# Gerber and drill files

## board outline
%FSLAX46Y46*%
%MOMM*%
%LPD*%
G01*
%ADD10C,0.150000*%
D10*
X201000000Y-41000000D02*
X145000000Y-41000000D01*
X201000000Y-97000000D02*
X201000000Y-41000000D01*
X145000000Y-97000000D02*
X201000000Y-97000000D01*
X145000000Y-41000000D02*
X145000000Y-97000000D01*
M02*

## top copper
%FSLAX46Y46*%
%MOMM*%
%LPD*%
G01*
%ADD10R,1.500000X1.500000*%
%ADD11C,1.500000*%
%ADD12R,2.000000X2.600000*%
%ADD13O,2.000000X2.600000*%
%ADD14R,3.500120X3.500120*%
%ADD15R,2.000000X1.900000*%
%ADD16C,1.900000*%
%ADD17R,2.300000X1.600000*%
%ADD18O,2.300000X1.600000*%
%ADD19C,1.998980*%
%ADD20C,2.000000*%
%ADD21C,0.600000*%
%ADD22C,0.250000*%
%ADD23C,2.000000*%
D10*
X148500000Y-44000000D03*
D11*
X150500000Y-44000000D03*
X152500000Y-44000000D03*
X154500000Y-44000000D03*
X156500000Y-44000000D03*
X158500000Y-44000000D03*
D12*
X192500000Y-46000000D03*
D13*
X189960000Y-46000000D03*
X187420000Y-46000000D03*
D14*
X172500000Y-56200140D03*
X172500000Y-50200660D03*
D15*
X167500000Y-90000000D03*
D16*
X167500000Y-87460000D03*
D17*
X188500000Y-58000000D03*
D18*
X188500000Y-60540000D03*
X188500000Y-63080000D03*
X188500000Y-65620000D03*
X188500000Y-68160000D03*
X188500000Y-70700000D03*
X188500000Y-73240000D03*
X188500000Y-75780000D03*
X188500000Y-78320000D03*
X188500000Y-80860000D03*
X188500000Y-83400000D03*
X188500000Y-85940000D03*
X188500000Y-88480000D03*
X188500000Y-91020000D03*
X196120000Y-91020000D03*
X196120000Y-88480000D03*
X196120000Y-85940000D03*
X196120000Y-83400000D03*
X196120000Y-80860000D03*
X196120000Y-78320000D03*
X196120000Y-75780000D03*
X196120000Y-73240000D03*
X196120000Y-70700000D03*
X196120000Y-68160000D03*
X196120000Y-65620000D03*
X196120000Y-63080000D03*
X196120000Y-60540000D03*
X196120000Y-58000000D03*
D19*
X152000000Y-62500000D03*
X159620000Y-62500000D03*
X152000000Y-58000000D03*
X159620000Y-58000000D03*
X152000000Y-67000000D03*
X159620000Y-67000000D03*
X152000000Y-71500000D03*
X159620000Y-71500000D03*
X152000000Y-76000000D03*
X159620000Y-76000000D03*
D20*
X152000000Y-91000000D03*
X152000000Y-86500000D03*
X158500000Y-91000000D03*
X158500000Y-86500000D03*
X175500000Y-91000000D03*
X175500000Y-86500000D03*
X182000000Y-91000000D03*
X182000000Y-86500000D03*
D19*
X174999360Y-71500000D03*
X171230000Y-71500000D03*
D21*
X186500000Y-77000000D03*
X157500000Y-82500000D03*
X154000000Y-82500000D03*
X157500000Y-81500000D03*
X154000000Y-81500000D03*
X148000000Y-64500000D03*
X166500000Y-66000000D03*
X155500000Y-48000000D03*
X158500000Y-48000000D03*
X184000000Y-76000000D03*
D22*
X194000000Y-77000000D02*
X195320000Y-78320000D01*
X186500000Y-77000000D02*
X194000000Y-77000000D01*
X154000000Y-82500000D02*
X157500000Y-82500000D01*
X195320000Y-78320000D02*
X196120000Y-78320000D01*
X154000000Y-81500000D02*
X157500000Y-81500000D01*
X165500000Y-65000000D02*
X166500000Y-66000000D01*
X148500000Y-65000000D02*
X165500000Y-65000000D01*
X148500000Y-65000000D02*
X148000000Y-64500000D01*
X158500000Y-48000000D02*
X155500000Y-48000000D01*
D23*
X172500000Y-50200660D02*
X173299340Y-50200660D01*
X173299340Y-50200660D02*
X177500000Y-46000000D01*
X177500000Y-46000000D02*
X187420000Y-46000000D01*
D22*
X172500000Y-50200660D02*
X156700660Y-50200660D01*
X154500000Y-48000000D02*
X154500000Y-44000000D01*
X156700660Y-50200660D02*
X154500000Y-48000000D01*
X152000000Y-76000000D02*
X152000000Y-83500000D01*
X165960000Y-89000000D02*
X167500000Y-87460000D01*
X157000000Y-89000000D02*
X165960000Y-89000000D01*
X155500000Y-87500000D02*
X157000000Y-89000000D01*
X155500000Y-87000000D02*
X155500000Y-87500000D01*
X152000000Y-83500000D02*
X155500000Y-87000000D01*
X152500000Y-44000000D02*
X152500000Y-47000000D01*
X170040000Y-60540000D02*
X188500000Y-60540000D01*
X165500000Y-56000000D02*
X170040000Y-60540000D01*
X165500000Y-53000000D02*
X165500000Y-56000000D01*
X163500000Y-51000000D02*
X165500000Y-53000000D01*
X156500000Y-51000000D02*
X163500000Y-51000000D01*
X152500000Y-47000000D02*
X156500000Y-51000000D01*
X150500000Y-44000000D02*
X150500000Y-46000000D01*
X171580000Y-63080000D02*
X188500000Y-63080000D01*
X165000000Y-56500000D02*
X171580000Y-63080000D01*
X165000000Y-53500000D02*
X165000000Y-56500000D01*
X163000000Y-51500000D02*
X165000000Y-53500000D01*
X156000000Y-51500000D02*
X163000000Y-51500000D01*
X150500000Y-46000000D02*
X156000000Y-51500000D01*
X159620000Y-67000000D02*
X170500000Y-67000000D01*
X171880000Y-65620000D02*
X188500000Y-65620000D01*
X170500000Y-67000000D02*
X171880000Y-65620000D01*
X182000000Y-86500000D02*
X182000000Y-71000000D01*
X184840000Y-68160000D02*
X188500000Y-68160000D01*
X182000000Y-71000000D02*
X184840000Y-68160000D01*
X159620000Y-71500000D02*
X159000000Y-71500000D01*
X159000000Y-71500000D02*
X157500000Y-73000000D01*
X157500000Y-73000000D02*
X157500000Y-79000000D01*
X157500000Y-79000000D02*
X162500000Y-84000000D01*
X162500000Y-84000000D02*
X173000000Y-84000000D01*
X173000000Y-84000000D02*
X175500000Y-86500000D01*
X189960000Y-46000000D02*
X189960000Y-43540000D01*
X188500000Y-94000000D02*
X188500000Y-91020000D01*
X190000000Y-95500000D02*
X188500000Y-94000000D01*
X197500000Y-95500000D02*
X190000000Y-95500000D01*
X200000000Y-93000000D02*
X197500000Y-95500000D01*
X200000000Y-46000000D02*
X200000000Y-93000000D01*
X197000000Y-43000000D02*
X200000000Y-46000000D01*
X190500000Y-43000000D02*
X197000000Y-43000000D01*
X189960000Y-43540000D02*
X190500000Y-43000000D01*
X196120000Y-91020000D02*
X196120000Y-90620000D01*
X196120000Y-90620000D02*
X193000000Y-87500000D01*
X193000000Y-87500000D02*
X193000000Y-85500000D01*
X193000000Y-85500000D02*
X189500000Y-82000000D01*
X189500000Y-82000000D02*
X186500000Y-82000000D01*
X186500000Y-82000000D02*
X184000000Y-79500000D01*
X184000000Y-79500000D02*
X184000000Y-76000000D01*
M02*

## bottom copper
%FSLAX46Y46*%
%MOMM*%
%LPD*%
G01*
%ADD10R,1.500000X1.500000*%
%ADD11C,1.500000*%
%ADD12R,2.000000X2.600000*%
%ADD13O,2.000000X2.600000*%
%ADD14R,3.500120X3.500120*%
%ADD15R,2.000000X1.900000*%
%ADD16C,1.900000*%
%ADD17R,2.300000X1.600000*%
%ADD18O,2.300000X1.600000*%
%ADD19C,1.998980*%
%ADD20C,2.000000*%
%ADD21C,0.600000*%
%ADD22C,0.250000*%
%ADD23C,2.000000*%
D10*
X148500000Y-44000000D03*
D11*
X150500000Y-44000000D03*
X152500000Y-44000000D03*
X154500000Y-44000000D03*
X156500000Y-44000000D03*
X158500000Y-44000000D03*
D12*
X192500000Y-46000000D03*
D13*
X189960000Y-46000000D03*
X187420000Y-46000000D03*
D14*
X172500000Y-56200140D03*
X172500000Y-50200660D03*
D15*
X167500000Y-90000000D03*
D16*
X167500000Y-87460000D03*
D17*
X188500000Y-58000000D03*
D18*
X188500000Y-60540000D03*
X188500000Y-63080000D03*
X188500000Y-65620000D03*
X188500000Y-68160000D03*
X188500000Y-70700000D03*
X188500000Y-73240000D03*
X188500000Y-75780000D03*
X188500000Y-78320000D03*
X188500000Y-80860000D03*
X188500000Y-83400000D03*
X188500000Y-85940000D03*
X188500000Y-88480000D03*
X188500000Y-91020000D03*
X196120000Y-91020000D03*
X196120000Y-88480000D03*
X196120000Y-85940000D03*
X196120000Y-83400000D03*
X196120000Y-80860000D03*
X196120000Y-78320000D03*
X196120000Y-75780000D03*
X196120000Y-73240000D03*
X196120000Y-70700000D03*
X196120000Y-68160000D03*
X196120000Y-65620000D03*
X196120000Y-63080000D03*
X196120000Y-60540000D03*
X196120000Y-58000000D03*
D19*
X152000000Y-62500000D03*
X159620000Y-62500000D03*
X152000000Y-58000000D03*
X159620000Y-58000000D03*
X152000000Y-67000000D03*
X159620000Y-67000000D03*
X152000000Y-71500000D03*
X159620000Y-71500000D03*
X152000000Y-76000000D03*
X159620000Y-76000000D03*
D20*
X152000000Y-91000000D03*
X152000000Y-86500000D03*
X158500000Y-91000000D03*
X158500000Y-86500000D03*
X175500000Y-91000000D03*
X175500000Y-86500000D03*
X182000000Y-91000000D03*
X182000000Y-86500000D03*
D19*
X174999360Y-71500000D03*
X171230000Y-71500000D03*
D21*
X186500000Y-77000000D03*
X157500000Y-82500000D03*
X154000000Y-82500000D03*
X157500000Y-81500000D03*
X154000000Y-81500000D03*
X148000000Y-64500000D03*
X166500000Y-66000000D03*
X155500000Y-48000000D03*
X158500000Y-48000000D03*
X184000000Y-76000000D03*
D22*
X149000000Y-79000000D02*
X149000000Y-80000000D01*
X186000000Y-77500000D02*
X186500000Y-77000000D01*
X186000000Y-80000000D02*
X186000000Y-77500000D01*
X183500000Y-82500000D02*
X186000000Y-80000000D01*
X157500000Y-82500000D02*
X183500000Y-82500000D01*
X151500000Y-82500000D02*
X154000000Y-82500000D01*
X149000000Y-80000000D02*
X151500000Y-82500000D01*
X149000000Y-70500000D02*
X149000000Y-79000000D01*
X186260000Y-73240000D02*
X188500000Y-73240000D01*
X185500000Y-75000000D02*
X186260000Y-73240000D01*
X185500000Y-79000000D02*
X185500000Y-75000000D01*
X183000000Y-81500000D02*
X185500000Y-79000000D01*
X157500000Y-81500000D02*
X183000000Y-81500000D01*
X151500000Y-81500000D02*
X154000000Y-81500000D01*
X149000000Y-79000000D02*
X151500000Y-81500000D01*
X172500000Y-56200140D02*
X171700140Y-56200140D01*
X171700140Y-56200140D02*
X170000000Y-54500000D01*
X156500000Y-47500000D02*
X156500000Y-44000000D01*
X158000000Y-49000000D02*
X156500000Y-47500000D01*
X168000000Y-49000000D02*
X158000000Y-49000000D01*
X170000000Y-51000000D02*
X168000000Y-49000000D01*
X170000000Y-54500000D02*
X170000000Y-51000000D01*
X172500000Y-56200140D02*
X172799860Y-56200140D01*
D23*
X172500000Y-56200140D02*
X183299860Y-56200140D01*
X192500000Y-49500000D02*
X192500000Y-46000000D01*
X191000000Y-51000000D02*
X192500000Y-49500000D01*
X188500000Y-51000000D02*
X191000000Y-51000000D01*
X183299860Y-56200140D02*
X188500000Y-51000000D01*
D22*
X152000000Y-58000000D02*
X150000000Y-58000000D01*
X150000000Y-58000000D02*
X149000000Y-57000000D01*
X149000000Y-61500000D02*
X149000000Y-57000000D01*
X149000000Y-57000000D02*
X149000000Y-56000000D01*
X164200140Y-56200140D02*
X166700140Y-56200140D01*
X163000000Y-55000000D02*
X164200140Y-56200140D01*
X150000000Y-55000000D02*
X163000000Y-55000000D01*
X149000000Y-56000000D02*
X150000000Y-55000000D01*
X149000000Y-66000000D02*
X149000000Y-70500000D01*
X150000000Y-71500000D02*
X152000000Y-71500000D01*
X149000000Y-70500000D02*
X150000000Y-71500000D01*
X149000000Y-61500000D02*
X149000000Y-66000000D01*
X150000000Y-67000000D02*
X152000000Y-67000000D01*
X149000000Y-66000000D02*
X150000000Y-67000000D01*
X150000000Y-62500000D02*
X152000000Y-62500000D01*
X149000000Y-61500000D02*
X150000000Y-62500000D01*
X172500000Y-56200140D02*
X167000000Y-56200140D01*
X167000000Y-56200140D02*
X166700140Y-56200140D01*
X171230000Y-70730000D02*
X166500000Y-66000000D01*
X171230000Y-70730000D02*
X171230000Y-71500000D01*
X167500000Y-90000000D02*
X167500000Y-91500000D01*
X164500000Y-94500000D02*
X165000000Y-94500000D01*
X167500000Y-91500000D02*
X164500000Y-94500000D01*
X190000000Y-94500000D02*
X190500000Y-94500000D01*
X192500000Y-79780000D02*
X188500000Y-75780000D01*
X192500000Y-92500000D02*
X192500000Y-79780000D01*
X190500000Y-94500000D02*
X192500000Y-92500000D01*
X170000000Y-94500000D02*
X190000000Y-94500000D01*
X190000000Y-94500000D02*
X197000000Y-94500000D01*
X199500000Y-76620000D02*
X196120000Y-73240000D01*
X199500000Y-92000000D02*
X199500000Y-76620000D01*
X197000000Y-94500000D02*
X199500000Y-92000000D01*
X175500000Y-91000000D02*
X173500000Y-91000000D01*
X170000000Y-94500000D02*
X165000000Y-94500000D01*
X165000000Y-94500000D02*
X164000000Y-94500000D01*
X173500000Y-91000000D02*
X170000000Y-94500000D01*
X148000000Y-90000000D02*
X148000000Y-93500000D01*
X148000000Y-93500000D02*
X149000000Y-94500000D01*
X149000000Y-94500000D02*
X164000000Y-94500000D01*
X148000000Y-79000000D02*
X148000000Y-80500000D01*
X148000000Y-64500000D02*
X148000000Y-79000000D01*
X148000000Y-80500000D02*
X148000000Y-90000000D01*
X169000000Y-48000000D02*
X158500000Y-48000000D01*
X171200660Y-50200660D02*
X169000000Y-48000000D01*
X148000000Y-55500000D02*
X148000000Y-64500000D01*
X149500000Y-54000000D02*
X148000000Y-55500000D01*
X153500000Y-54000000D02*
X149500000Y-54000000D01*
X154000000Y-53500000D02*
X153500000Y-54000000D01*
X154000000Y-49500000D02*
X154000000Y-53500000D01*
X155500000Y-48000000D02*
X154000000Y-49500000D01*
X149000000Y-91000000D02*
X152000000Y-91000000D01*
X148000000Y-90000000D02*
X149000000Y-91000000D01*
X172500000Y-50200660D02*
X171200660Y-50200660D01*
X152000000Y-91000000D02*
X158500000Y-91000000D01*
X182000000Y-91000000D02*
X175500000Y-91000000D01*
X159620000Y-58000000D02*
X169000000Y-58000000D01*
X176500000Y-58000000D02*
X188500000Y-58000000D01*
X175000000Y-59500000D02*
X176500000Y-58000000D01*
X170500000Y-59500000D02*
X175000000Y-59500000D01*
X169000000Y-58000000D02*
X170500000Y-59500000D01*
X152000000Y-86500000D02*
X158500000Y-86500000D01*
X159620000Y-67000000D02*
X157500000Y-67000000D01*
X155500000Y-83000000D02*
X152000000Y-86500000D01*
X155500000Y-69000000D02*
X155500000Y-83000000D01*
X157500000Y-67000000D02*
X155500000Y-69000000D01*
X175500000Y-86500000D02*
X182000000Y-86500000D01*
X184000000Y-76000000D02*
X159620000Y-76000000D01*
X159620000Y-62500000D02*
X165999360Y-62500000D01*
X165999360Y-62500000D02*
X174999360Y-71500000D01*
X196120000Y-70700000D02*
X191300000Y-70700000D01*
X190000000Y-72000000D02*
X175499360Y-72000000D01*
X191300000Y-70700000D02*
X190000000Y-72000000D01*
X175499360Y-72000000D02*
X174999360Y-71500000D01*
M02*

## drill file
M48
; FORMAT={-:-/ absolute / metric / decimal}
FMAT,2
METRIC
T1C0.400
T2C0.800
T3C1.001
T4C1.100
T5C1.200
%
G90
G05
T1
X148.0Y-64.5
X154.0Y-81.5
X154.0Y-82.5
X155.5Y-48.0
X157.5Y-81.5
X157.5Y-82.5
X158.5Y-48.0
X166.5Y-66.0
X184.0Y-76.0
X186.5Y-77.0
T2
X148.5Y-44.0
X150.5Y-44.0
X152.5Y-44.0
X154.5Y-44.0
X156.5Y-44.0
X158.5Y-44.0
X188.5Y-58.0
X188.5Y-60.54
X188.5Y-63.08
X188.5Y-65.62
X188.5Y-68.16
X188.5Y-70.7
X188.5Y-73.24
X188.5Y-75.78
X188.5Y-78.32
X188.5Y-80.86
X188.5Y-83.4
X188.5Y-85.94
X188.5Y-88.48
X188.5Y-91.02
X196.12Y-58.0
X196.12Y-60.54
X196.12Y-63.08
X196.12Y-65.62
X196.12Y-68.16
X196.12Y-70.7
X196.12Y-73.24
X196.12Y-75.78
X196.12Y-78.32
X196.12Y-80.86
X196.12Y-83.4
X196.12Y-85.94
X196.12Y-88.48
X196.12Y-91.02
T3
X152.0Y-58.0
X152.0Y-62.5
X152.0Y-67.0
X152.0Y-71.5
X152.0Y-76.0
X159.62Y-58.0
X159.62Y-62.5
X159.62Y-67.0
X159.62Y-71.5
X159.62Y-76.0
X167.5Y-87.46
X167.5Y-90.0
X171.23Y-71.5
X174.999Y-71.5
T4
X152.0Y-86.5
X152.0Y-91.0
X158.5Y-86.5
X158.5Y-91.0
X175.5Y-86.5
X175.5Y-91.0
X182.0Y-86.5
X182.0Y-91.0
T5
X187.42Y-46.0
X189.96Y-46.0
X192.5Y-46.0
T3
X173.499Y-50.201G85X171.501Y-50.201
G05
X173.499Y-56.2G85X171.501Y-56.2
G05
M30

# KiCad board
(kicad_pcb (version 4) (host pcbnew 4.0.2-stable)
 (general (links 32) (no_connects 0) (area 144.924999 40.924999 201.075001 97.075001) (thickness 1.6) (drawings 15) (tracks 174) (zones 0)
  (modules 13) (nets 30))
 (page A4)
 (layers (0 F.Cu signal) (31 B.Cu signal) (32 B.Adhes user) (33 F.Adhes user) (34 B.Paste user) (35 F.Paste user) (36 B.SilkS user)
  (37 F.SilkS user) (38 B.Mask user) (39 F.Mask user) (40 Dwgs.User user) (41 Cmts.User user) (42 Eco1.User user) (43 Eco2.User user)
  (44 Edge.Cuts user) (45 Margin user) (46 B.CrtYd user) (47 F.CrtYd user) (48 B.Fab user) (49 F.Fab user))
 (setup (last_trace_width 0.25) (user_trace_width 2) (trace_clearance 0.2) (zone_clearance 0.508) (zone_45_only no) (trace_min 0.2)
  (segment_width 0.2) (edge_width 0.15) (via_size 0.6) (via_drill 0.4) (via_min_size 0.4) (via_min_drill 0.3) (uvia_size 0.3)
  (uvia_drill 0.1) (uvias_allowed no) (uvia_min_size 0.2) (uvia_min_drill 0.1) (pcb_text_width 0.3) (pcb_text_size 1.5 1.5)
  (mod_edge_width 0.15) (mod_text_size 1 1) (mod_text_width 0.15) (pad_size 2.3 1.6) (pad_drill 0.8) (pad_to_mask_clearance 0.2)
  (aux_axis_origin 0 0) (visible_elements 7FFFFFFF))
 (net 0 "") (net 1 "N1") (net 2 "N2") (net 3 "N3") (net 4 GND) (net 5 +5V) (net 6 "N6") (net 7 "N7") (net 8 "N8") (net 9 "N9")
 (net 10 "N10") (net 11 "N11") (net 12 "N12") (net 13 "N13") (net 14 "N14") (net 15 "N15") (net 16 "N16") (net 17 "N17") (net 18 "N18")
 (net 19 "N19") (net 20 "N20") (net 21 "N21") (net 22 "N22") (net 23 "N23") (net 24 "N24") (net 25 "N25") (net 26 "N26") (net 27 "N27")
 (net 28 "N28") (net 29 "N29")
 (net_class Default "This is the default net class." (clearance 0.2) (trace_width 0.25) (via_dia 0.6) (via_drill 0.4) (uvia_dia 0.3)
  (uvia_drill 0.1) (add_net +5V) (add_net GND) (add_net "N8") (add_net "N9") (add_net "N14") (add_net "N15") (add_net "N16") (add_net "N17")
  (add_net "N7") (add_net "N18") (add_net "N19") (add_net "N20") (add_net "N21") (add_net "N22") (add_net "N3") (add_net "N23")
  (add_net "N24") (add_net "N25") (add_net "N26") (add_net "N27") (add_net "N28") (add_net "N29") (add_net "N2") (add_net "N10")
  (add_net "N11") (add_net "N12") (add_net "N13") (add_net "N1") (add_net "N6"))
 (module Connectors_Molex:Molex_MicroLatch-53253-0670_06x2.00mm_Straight (layer F.Cu) (at 148.5 44)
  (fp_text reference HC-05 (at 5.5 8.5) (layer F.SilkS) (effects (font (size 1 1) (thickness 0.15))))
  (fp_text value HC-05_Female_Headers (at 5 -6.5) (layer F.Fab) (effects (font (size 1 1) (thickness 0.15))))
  (pad 1 thru_hole rect (at 0 0) (size 1.5 1.5) (drill 0.8) (layers *.Cu *.Mask) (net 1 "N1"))
  (pad 2 thru_hole circle (at 2 0) (size 1.5 1.5) (drill 0.8) (layers *.Cu *.Mask) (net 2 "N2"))
  (pad 3 thru_hole circle (at 4 0) (size 1.5 1.5) (drill 0.8) (layers *.Cu *.Mask) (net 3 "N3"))
  (pad 4 thru_hole circle (at 6 0) (size 1.5 1.5) (drill 0.8) (layers *.Cu *.Mask) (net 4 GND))
  (pad 5 thru_hole circle (at 8 0) (size 1.5 1.5) (drill 0.8) (layers *.Cu *.Mask) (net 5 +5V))
  (pad 6 thru_hole circle (at 10 0) (size 1.5 1.5) (drill 0.8) (layers *.Cu *.Mask) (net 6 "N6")))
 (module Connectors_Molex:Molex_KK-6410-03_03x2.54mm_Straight (layer F.Cu) (at 192.5 46 180)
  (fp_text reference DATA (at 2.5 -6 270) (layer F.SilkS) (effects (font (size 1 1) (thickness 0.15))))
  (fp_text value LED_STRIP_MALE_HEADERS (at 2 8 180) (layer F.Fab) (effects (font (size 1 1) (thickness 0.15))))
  (pad 1 thru_hole rect (at 0 0 180) (size 2 2.6) (drill 1.2) (layers *.Cu *.Mask F.SilkS) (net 5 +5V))
  (pad 2 thru_hole oval (at 2.54 0 180) (size 2 2.6) (drill 1.2) (layers *.Cu *.Mask F.SilkS) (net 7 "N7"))
  (pad 3 thru_hole oval (at 5.08 0 180) (size 2 2.6) (drill 1.2) (layers *.Cu *.Mask F.SilkS) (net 4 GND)))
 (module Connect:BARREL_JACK (layer F.Cu) (at 172.5 50 270)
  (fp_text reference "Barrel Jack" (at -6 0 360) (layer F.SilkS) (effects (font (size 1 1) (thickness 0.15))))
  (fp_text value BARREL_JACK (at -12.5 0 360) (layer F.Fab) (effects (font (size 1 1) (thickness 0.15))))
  (pad 1 thru_hole rect (at 6.20014 0 270) (size 3.50012 3.50012) (drill oval 1.00076 2.99974) (layers *.Cu *.Mask F.SilkS) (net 5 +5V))
  (pad 2 thru_hole rect (at 0.20066 0 270) (size 3.50012 3.50012) (drill oval 1.00076 2.99974) (layers *.Cu *.Mask F.SilkS) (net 4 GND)))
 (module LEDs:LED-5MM (layer F.Cu) (at 167.5 90 90)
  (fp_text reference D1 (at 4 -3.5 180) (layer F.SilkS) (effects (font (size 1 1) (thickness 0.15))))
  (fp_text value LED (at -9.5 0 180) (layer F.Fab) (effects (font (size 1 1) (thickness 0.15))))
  (pad 1 thru_hole rect (at 0 0 180) (size 2 1.9) (drill 1.00076) (layers *.Cu *.Mask F.SilkS) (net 4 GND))
  (pad 2 thru_hole circle (at 2.54 0 90) (size 1.9 1.9) (drill 1.00076) (layers *.Cu *.Mask F.SilkS) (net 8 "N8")))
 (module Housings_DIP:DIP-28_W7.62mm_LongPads (layer F.Cu) (at 188.5 58)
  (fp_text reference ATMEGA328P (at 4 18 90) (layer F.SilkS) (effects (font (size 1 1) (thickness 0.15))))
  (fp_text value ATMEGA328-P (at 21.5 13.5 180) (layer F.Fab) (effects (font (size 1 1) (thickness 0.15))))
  (pad 1 thru_hole rect (at 0 0) (size 2.3 1.6) (drill 0.8) (layers *.Cu *.Mask F.SilkS) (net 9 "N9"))
  (pad 2 thru_hole oval (at 0 2.54) (size 2.3 1.6) (drill 0.8) (layers *.Cu *.Mask F.SilkS) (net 3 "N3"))
  (pad 3 thru_hole oval (at 0 5.08) (size 2.3 1.6) (drill 0.8) (layers *.Cu *.Mask F.SilkS) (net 2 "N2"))
  (pad 4 thru_hole oval (at 0 7.62) (size 2.3 1.6) (drill 0.8) (layers *.Cu *.Mask F.SilkS) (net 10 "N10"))
  (pad 5 thru_hole oval (at 0 10.16) (size 2.3 1.6) (drill 0.8) (layers *.Cu *.Mask F.SilkS) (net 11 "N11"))
  (pad 6 thru_hole oval (at 0 12.7) (size 2.3 1.6) (drill 0.8) (layers *.Cu *.Mask F.SilkS) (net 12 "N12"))
  (pad 7 thru_hole oval (at 0 15.24) (size 2.3 1.6) (drill 0.8) (layers *.Cu *.Mask F.SilkS) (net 5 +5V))
  (pad 8 thru_hole oval (at 0 17.78) (size 2.3 1.6) (drill 0.8) (layers *.Cu *.Mask F.SilkS) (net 4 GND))
  (pad 9 thru_hole oval (at 0 20.32) (size 2.3 1.6) (drill 0.8) (layers *.Cu *.Mask F.SilkS) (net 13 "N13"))
  (pad 10 thru_hole oval (at 0 22.86) (size 2.3 1.6) (drill 0.8) (layers *.Cu *.Mask F.SilkS) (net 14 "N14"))
  (pad 11 thru_hole oval (at 0 25.4) (size 2.3 1.6) (drill 0.8) (layers *.Cu *.Mask F.SilkS) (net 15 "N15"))
  (pad 12 thru_hole oval (at 0 27.94) (size 2.3 1.6) (drill 0.8) (layers *.Cu *.Mask F.SilkS) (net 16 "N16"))
  (pad 13 thru_hole oval (at 0 30.48) (size 2.3 1.6) (drill 0.8) (layers *.Cu *.Mask F.SilkS) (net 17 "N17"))
  (pad 14 thru_hole oval (at 0 33.02) (size 2.3 1.6) (drill 0.8) (layers *.Cu *.Mask F.SilkS) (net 7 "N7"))
  (pad 15 thru_hole oval (at 7.62 33.02) (size 2.3 1.6) (drill 0.8) (layers *.Cu *.Mask F.SilkS) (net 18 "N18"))
  (pad 16 thru_hole oval (at 7.62 30.48) (size 2.3 1.6) (drill 0.8) (layers *.Cu *.Mask F.SilkS) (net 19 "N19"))
  (pad 17 thru_hole oval (at 7.62 27.94) (size 2.3 1.6) (drill 0.8) (layers *.Cu *.Mask F.SilkS) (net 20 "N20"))
  (pad 18 thru_hole oval (at 7.62 25.4) (size 2.3 1.6) (drill 0.8) (layers *.Cu *.Mask F.SilkS) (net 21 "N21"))
  (pad 19 thru_hole oval (at 7.62 22.86) (size 2.3 1.6) (drill 0.8) (layers *.Cu *.Mask F.SilkS) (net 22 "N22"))
  (pad 20 thru_hole oval (at 7.62 20.32) (size 2.3 1.6) (drill 0.8) (layers *.Cu *.Mask F.SilkS) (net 5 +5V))
  (pad 21 thru_hole oval (at 7.62 17.78) (size 2.3 1.6) (drill 0.8) (layers *.Cu *.Mask F.SilkS) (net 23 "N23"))
  (pad 22 thru_hole oval (at 7.62 15.24) (size 2.3 1.6) (drill 0.8) (layers *.Cu *.Mask F.SilkS) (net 4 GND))
  (pad 23 thru_hole oval (at 7.62 12.7) (size 2.3 1.6) (drill 0.8) (layers *.Cu *.Mask F.SilkS) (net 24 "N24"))
  (pad 24 thru_hole oval (at 7.62 10.16) (size 2.3 1.6) (drill 0.8) (layers *.Cu *.Mask F.SilkS) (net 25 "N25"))
  (pad 25 thru_hole oval (at 7.62 7.62) (size 2.3 1.6) (drill 0.8) (layers *.Cu *.Mask F.SilkS) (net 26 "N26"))
  (pad 26 thru_hole oval (at 7.62 5.08) (size 2.3 1.6) (drill 0.8) (layers *.Cu *.Mask F.SilkS) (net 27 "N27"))
  (pad 27 thru_hole oval (at 7.62 2.54) (size 2.3 1.6) (drill 0.8) (layers *.Cu *.Mask F.SilkS) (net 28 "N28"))
  (pad 28 thru_hole oval (at 7.62 0) (size 2.3 1.6) (drill 0.8) (layers *.Cu *.Mask F.SilkS) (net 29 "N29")))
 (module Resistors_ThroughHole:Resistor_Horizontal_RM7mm (layer F.Cu) (at 152 62.5)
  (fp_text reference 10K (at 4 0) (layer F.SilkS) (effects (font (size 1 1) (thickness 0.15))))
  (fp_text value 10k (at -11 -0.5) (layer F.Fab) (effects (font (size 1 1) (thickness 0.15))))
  (pad 1 thru_hole circle (at 0 0) (size 1.99898 1.99898) (drill 1.00076) (layers *.Cu *.SilkS *.Mask) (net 5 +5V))
  (pad 2 thru_hole circle (at 7.62 0) (size 1.99898 1.99898) (drill 1.00076) (layers *.Cu *.SilkS *.Mask) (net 24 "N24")))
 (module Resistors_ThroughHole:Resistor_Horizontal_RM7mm (layer F.Cu) (at 152 58)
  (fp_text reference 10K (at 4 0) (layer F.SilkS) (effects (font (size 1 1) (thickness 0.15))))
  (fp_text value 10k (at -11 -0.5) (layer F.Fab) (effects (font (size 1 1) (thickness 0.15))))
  (pad 1 thru_hole circle (at 0 0) (size 1.99898 1.99898) (drill 1.00076) (layers *.Cu *.SilkS *.Mask) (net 5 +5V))
  (pad 2 thru_hole circle (at 7.62 0) (size 1.99898 1.99898) (drill 1.00076) (layers *.Cu *.SilkS *.Mask) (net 9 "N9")))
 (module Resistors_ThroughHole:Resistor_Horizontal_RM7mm (layer F.Cu) (at 152 67)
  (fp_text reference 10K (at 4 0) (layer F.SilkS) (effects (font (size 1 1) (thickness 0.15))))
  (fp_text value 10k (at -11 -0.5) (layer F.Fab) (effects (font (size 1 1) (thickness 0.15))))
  (pad 1 thru_hole circle (at 0 0) (size 1.99898 1.99898) (drill 1.00076) (layers *.Cu *.SilkS *.Mask) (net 5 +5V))
  (pad 2 thru_hole circle (at 7.62 0) (size 1.99898 1.99898) (drill 1.00076) (layers *.Cu *.SilkS *.Mask) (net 10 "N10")))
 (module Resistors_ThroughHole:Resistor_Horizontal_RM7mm (layer F.Cu) (at 152 71.5)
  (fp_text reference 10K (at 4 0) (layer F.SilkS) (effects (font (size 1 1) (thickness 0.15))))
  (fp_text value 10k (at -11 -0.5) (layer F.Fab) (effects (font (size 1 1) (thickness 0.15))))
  (pad 1 thru_hole circle (at 0 0) (size 1.99898 1.99898) (drill 1.00076) (layers *.Cu *.SilkS *.Mask) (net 5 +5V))
  (pad 2 thru_hole circle (at 7.62 0) (size 1.99898 1.99898) (drill 1.00076) (layers *.Cu *.SilkS *.Mask) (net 11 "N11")))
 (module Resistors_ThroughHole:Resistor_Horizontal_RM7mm (layer F.Cu) (at 152 76)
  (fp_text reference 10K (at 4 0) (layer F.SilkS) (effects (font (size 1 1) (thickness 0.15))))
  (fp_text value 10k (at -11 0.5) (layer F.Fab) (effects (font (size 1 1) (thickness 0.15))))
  (pad 1 thru_hole circle (at 0 0) (size 1.99898 1.99898) (drill 1.00076) (layers *.Cu *.SilkS *.Mask) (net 8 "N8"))
  (pad 2 thru_hole circle (at 7.62 0) (size 1.99898 1.99898) (drill 1.00076) (layers *.Cu *.SilkS *.Mask) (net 18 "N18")))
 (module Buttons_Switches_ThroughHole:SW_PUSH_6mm (layer F.Cu) (at 152 86.5)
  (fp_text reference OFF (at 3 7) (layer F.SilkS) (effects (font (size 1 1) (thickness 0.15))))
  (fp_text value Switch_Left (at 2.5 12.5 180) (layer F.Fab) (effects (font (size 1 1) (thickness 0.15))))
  (pad 2 thru_hole circle (at 0 4.5 90) (size 2 2) (drill 1.1) (layers *.Cu *.Mask) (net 4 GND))
  (pad 1 thru_hole circle (at 0 0 90) (size 2 2) (drill 1.1) (layers *.Cu *.Mask) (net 10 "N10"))
  (pad 2 thru_hole circle (at 6.5 4.5 90) (size 2 2) (drill 1.1) (layers *.Cu *.Mask) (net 4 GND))
  (pad 1 thru_hole circle (at 6.5 0 90) (size 2 2) (drill 1.1) (layers *.Cu *.Mask) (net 10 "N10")))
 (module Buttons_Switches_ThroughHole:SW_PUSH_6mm (layer F.Cu) (at 175.5 86.5)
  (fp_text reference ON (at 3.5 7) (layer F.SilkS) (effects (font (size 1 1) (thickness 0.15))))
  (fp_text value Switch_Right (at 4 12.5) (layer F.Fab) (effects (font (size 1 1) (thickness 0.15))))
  (pad 2 thru_hole circle (at 0 4.5 90) (size 2 2) (drill 1.1) (layers *.Cu *.Mask) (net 4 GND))
  (pad 1 thru_hole circle (at 0 0 90) (size 2 2) (drill 1.1) (layers *.Cu *.Mask) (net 11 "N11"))
  (pad 2 thru_hole circle (at 6.5 4.5 90) (size 2 2) (drill 1.1) (layers *.Cu *.Mask) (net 4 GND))
  (pad 1 thru_hole circle (at 6.5 0 90) (size 2 2) (drill 1.1) (layers *.Cu *.Mask) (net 11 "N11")))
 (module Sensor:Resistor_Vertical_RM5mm (layer F.Cu) (at 172.5 71.5 180)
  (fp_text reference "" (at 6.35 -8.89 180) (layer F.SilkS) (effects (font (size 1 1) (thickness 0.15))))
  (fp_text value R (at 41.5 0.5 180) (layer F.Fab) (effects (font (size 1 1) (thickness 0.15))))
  (pad 1 thru_hole circle (at -2.49936 0 180) (size 1.99898 1.99898) (drill 1.00076) (layers *.Cu *.Mask B.SilkS) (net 24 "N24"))
  (pad 2 thru_hole circle (at 1.27 0 180) (size 1.99898 1.99898) (drill 1.00076) (layers *.Cu *.SilkS *.Mask) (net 4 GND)))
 (gr_line (start 201 41) (end 145 41) (angle 90) (layer Edge.Cuts) (width 0.15))
 (gr_line (start 201 97) (end 201 41) (angle 90) (layer Edge.Cuts) (width 0.15))
 (gr_line (start 145 97) (end 201 97) (angle 90) (layer Edge.Cuts) (width 0.15))
 (gr_line (start 145 41) (end 145 97) (angle 90) (layer Edge.Cuts) (width 0.15))
 (segment (start 149 79) (end 149 80) (width 0.25) (layer B.Cu) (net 5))
 (segment (start 194 77) (end 195.32 78.32) (width 0.25) (layer F.Cu) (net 5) (status 20))
 (segment (start 186.5 77) (end 194 77) (width 0.25) (layer F.Cu) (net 5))
 (via (at 186.5 77) (size 0.6) (drill 0.4) (layers F.Cu B.Cu) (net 5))
 (segment (start 186 77.5) (end 186.5 77) (width 0.25) (layer B.Cu) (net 5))
 (segment (start 186 80) (end 186 77.5) (width 0.25) (layer B.Cu) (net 5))
 (segment (start 183.5 82.5) (end 186 80) (width 0.25) (layer B.Cu) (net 5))
 (segment (start 157.5 82.5) (end 183.5 82.5) (width 0.25) (layer B.Cu) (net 5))
 (via (at 157.5 82.5) (size 0.6) (drill 0.4) (layers F.Cu B.Cu) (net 5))
 (segment (start 154 82.5) (end 157.5 82.5) (width 0.25) (layer F.Cu) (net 5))
 (via (at 154 82.5) (size 0.6) (drill 0.4) (layers F.Cu B.Cu) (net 5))
 (segment (start 151.5 82.5) (end 154 82.5) (width 0.25) (layer B.Cu) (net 5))
 (segment (start 149 80) (end 151.5 82.5) (width 0.25) (layer B.Cu) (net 5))
 (segment (start 195.32 78.32) (end 196.12 78.32) (width 0.25) (layer F.Cu) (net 5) (status 30))
 (segment (start 149 70.5) (end 149 79) (width 0.25) (layer B.Cu) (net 5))
 (segment (start 186.26 73.24) (end 188.5 73.24) (width 0.25) (layer B.Cu) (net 5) (status 20))
 (segment (start 185.5 75) (end 186.26 73.24) (width 0.25) (layer B.Cu) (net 5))
 (segment (start 185.5 79) (end 185.5 75) (width 0.25) (layer B.Cu) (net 5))
 (segment (start 183 81.5) (end 185.5 79) (width 0.25) (layer B.Cu) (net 5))
 (segment (start 157.5 81.5) (end 183 81.5) (width 0.25) (layer B.Cu) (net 5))
 (via (at 157.5 81.5) (size 0.6) (drill 0.4) (layers F.Cu B.Cu) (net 5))
 (segment (start 154 81.5) (end 157.5 81.5) (width 0.25) (layer F.Cu) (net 5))
 (via (at 154 81.5) (size 0.6) (drill 0.4) (layers F.Cu B.Cu) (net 5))
 (segment (start 151.5 81.5) (end 154 81.5) (width 0.25) (layer B.Cu) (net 5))
 (segment (start 149 79) (end 151.5 81.5) (width 0.25) (layer B.Cu) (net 5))
 (segment (start 172.5 56.20014) (end 171.70014 56.20014) (width 0.25) (layer B.Cu) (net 5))
 (segment (start 171.70014 56.20014) (end 170 54.5) (width 0.25) (layer B.Cu) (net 5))
 (segment (start 156.5 47.5) (end 156.5 44) (width 0.25) (layer B.Cu) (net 5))
 (segment (start 158 49) (end 156.5 47.5) (width 0.25) (layer B.Cu) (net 5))
 (segment (start 168 49) (end 158 49) (width 0.25) (layer B.Cu) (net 5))
 (segment (start 170 51) (end 168 49) (width 0.25) (layer B.Cu) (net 5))
 (segment (start 170 54.5) (end 170 51) (width 0.25) (layer B.Cu) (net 5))
 (segment (start 172.5 56.20014) (end 172.79986 56.20014) (width 0.25) (layer B.Cu) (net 5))
 (segment (start 172.5 56.20014) (end 183.29986 56.20014) (width 2) (layer B.Cu) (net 5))
 (segment (start 192.5 49.5) (end 192.5 46) (width 2) (layer B.Cu) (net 5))
 (segment (start 191 51) (end 192.5 49.5) (width 2) (layer B.Cu) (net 5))
 (segment (start 188.5 51) (end 191 51) (width 2) (layer B.Cu) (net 5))
 (segment (start 183.29986 56.20014) (end 188.5 51) (width 2) (layer B.Cu) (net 5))
 (segment (start 152 58) (end 150 58) (width 0.25) (layer B.Cu) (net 5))
 (segment (start 150 58) (end 149 57) (width 0.25) (layer B.Cu) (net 5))
 (segment (start 149 61.5) (end 149 57) (width 0.25) (layer B.Cu) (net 5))
 (segment (start 149 57) (end 149 56) (width 0.25) (layer B.Cu) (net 5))
 (segment (start 164.20014 56.20014) (end 166.70014 56.20014) (width 0.25) (layer B.Cu) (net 5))
 (segment (start 163 55) (end 164.20014 56.20014) (width 0.25) (layer B.Cu) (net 5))
 (segment (start 150 55) (end 163 55) (width 0.25) (layer B.Cu) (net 5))
 (segment (start 149 56) (end 150 55) (width 0.25) (layer B.Cu) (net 5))
 (segment (start 149 66) (end 149 70.5) (width 0.25) (layer B.Cu) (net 5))
 (segment (start 150 71.5) (end 152 71.5) (width 0.25) (layer B.Cu) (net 5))
 (segment (start 149 70.5) (end 150 71.5) (width 0.25) (layer B.Cu) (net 5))
 (segment (start 149 61.5) (end 149 66) (width 0.25) (layer B.Cu) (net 5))
 (segment (start 150 67) (end 152 67) (width 0.25) (layer B.Cu) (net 5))
 (segment (start 149 66) (end 150 67) (width 0.25) (layer B.Cu) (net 5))
 (segment (start 150 62.5) (end 152 62.5) (width 0.25) (layer B.Cu) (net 5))
 (segment (start 149 61.5) (end 150 62.5) (width 0.25) (layer B.Cu) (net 5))
 (segment (start 172.5 56.20014) (end 167 56.20014) (width 0.25) (layer B.Cu) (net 5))
 (segment (start 167 56.20014) (end 166.70014 56.20014) (width 0.25) (layer B.Cu) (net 5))
 (via (at 148 64.5) (size 0.6) (drill 0.4) (layers F.Cu B.Cu) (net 4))
 (segment (start 171.23 70.73) (end 166.5 66) (width 0.25) (layer B.Cu) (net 4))
 (via (at 166.5 66) (size 0.6) (drill 0.4) (layers F.Cu B.Cu) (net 4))
 (segment (start 165.5 65) (end 166.5 66) (width 0.25) (layer F.Cu) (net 4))
 (segment (start 148.5 65) (end 165.5 65) (width 0.25) (layer F.Cu) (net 4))
 (segment (start 148.5 65) (end 148 64.5) (width 0.25) (layer F.Cu) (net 4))
 (segment (start 171.23 70.73) (end 171.23 71.5) (width 0.25) (layer B.Cu) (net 4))
 (segment (start 167.5 90) (end 167.5 91.5) (width 0.25) (layer B.Cu) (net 4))
 (segment (start 164.5 94.5) (end 165 94.5) (width 0.25) (layer B.Cu) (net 4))
 (segment (start 167.5 91.5) (end 164.5 94.5) (width 0.25) (layer B.Cu) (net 4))
 (segment (start 190 94.5) (end 190.5 94.5) (width 0.25) (layer B.Cu) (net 4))
 (segment (start 192.5 79.78) (end 188.5 75.78) (width 0.25) (layer B.Cu) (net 4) (status 20))
 (segment (start 192.5 92.5) (end 192.5 79.78) (width 0.25) (layer B.Cu) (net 4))
 (segment (start 190.5 94.5) (end 192.5 92.5) (width 0.25) (layer B.Cu) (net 4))
 (segment (start 170 94.5) (end 190 94.5) (width 0.25) (layer B.Cu) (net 4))
 (segment (start 190 94.5) (end 197 94.5) (width 0.25) (layer B.Cu) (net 4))
 (segment (start 199.5 76.62) (end 196.12 73.24) (width 0.25) (layer B.Cu) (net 4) (status 20))
 (segment (start 199.5 92) (end 199.5 76.62) (width 0.25) (layer B.Cu) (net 4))
 (segment (start 197 94.5) (end 199.5 92) (width 0.25) (layer B.Cu) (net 4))
 (segment (start 175.5 91) (end 173.5 91) (width 0.25) (layer B.Cu) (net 4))
 (segment (start 170 94.5) (end 165 94.5) (width 0.25) (layer B.Cu) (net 4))
 (segment (start 165 94.5) (end 164 94.5) (width 0.25) (layer B.Cu) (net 4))
 (segment (start 173.5 91) (end 170 94.5) (width 0.25) (layer B.Cu) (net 4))
 (segment (start 148 90) (end 148 93.5) (width 0.25) (layer B.Cu) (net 4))
 (segment (start 148 93.5) (end 149 94.5) (width 0.25) (layer B.Cu) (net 4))
 (segment (start 149 94.5) (end 164 94.5) (width 0.25) (layer B.Cu) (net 4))
 (segment (start 148 79) (end 148 80.5) (width 0.25) (layer B.Cu) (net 4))
 (segment (start 148 64.5) (end 148 79) (width 0.25) (layer B.Cu) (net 4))
 (segment (start 148 80.5) (end 148 90) (width 0.25) (layer B.Cu) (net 4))
 (segment (start 169 48) (end 158.5 48) (width 0.25) (layer B.Cu) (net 4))
 (segment (start 171.20066 50.20066) (end 169 48) (width 0.25) (layer B.Cu) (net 4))
 (segment (start 148 55.5) (end 148 64.5) (width 0.25) (layer B.Cu) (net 4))
 (segment (start 149.5 54) (end 148 55.5) (width 0.25) (layer B.Cu) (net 4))
 (segment (start 153.5 54) (end 149.5 54) (width 0.25) (layer B.Cu) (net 4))
 (segment (start 154 53.5) (end 153.5 54) (width 0.25) (layer B.Cu) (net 4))
 (segment (start 154 49.5) (end 154 53.5) (width 0.25) (layer B.Cu) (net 4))
 (segment (start 155.5 48) (end 154 49.5) (width 0.25) (layer B.Cu) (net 4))
 (via (at 155.5 48) (size 0.6) (drill 0.4) (layers F.Cu B.Cu) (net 4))
 (segment (start 158.5 48) (end 155.5 48) (width 0.25) (layer F.Cu) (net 4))
 (via (at 158.5 48) (size 0.6) (drill 0.4) (layers F.Cu B.Cu) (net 4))
 (segment (start 149 91) (end 152 91) (width 0.25) (layer B.Cu) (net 4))
 (segment (start 148 90) (end 149 91) (width 0.25) (layer B.Cu) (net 4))
 (segment (start 172.5 50.20066) (end 171.20066 50.20066) (width 0.25) (layer B.Cu) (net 4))
 (segment (start 152 91) (end 158.5 91) (width 0.25) (layer B.Cu) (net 4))
 (segment (start 182 91) (end 175.5 91) (width 0.25) (layer B.Cu) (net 4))
 (segment (start 172.5 50.20066) (end 173.29934 50.20066) (width 2) (layer F.Cu) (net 4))
 (segment (start 173.29934 50.20066) (end 177.5 46) (width 2) (layer F.Cu) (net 4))
 (segment (start 177.5 46) (end 187.42 46) (width 2) (layer F.Cu) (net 4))
 (segment (start 172.5 50.20066) (end 156.70066 50.20066) (width 0.25) (layer F.Cu) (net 4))
 (segment (start 154.5 48) (end 154.5 44) (width 0.25) (layer F.Cu) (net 4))
 (segment (start 156.70066 50.20066) (end 154.5 48) (width 0.25) (layer F.Cu) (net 4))
 (segment (start 152 76) (end 152 83.5) (width 0.25) (layer F.Cu) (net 8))
 (segment (start 165.96 89) (end 167.5 87.46) (width 0.25) (layer F.Cu) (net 8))
 (segment (start 157 89) (end 165.96 89) (width 0.25) (layer F.Cu) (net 8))
 (segment (start 155.5 87.5) (end 157 89) (width 0.25) (layer F.Cu) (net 8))
 (segment (start 155.5 87) (end 155.5 87.5) (width 0.25) (layer F.Cu) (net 8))
 (segment (start 152 83.5) (end 155.5 87) (width 0.25) (layer F.Cu) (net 8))
 (segment (start 159.62 58) (end 169 58) (width 0.25) (layer B.Cu) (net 9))
 (segment (start 176.5 58) (end 188.5 58) (width 0.25) (layer B.Cu) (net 9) (status 20))
 (segment (start 175 59.5) (end 176.5 58) (width 0.25) (layer B.Cu) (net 9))
 (segment (start 170.5 59.5) (end 175 59.5) (width 0.25) (layer B.Cu) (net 9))
 (segment (start 169 58) (end 170.5 59.5) (width 0.25) (layer B.Cu) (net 9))
 (segment (start 152.5 44) (end 152.5 47) (width 0.25) (layer F.Cu) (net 3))
 (segment (start 170.04 60.54) (end 188.5 60.54) (width 0.25) (layer F.Cu) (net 3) (status 20))
 (segment (start 165.5 56) (end 170.04 60.54) (width 0.25) (layer F.Cu) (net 3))
 (segment (start 165.5 53) (end 165.5 56) (width 0.25) (layer F.Cu) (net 3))
 (segment (start 163.5 51) (end 165.5 53) (width 0.25) (layer F.Cu) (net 3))
 (segment (start 156.5 51) (end 163.5 51) (width 0.25) (layer F.Cu) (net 3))
 (segment (start 152.5 47) (end 156.5 51) (width 0.25) (layer F.Cu) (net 3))
 (segment (start 150.5 44) (end 150.5 46) (width 0.25) (layer F.Cu) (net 2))
 (segment (start 171.58 63.08) (end 188.5 63.08) (width 0.25) (layer F.Cu) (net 2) (status 20))
 (segment (start 165 56.5) (end 171.58 63.08) (width 0.25) (layer F.Cu) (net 2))
 (segment (start 165 53.5) (end 165 56.5) (width 0.25) (layer F.Cu) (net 2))
 (segment (start 163 51.5) (end 165 53.5) (width 0.25) (layer F.Cu) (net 2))
 (segment (start 156 51.5) (end 163 51.5) (width 0.25) (layer F.Cu) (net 2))
 (segment (start 150.5 46) (end 156 51.5) (width 0.25) (layer F.Cu) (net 2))
 (segment (start 159.62 67) (end 170.5 67) (width 0.25) (layer F.Cu) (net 10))
 (segment (start 171.88 65.62) (end 188.5 65.62) (width 0.25) (layer F.Cu) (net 10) (status 20))
 (segment (start 170.5 67) (end 171.88 65.62) (width 0.25) (layer F.Cu) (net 10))
 (segment (start 152 86.5) (end 158.5 86.5) (width 0.25) (layer B.Cu) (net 10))
 (segment (start 159.62 67) (end 157.5 67) (width 0.25) (layer B.Cu) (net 10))
 (segment (start 155.5 83) (end 152 86.5) (width 0.25) (layer B.Cu) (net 10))
 (segment (start 155.5 69) (end 155.5 83) (width 0.25) (layer B.Cu) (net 10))
 (segment (start 157.5 67) (end 155.5 69) (width 0.25) (layer B.Cu) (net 10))
 (segment (start 182 86.5) (end 182 71) (width 0.25) (layer F.Cu) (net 11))
 (segment (start 184.84 68.16) (end 188.5 68.16) (width 0.25) (layer F.Cu) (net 11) (status 20))
 (segment (start 182 71) (end 184.84 68.16) (width 0.25) (layer F.Cu) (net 11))
 (segment (start 159.62 71.5) (end 159 71.5) (width 0.25) (layer F.Cu) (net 11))
 (segment (start 159 71.5) (end 157.5 73) (width 0.25) (layer F.Cu) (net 11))
 (segment (start 157.5 73) (end 157.5 79) (width 0.25) (layer F.Cu) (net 11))
 (segment (start 157.5 79) (end 162.5 84) (width 0.25) (layer F.Cu) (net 11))
 (segment (start 162.5 84) (end 173 84) (width 0.25) (layer F.Cu) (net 11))
 (segment (start 173 84) (end 175.5 86.5) (width 0.25) (layer F.Cu) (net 11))
 (segment (start 175.5 86.5) (end 182 86.5) (width 0.25) (layer B.Cu) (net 11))
 (segment (start 189.96 46) (end 189.96 43.54) (width 0.25) (layer F.Cu) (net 7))
 (segment (start 188.5 94) (end 188.5 91.02) (width 0.25) (layer F.Cu) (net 7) (status 20))
 (segment (start 190 95.5) (end 188.5 94) (width 0.25) (layer F.Cu) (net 7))
 (segment (start 197.5 95.5) (end 190 95.5) (width 0.25) (layer F.Cu) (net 7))
 (segment (start 200 93) (end 197.5 95.5) (width 0.25) (layer F.Cu) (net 7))
 (segment (start 200 46) (end 200 93) (width 0.25) (layer F.Cu) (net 7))
 (segment (start 197 43) (end 200 46) (width 0.25) (layer F.Cu) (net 7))
 (segment (start 190.5 43) (end 197 43) (width 0.25) (layer F.Cu) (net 7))
 (segment (start 189.96 43.54) (end 190.5 43) (width 0.25) (layer F.Cu) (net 7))
 (segment (start 196.12 91.02) (end 196.12 90.62) (width 0.25) (layer F.Cu) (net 18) (status 30))
 (segment (start 196.12 90.62) (end 193 87.5) (width 0.25) (layer F.Cu) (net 18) (status 10))
 (segment (start 193 87.5) (end 193 85.5) (width 0.25) (layer F.Cu) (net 18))
 (segment (start 193 85.5) (end 189.5 82) (width 0.25) (layer F.Cu) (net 18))
 (segment (start 189.5 82) (end 186.5 82) (width 0.25) (layer F.Cu) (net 18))
 (segment (start 186.5 82) (end 184 79.5) (width 0.25) (layer F.Cu) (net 18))
 (segment (start 184 79.5) (end 184 76) (width 0.25) (layer F.Cu) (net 18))
 (via (at 184 76) (size 0.6) (drill 0.4) (layers F.Cu B.Cu) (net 18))
 (segment (start 184 76) (end 159.62 76) (width 0.25) (layer B.Cu) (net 18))
 (segment (start 159.62 62.5) (end 165.99936 62.5) (width 0.25) (layer B.Cu) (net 24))
 (segment (start 165.99936 62.5) (end 174.99936 71.5) (width 0.25) (layer B.Cu) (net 24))
 (segment (start 196.12 70.7) (end 191.3 70.7) (width 0.25) (layer B.Cu) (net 24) (status 10))
 (segment (start 190 72) (end 175.49936 72) (width 0.25) (layer B.Cu) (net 24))
 (segment (start 191.3 70.7) (end 190 72) (width 0.25) (layer B.Cu) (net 24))
 (segment (start 175.49936 72) (end 174.99936 71.5) (width 0.25) (layer B.Cu) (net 24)))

